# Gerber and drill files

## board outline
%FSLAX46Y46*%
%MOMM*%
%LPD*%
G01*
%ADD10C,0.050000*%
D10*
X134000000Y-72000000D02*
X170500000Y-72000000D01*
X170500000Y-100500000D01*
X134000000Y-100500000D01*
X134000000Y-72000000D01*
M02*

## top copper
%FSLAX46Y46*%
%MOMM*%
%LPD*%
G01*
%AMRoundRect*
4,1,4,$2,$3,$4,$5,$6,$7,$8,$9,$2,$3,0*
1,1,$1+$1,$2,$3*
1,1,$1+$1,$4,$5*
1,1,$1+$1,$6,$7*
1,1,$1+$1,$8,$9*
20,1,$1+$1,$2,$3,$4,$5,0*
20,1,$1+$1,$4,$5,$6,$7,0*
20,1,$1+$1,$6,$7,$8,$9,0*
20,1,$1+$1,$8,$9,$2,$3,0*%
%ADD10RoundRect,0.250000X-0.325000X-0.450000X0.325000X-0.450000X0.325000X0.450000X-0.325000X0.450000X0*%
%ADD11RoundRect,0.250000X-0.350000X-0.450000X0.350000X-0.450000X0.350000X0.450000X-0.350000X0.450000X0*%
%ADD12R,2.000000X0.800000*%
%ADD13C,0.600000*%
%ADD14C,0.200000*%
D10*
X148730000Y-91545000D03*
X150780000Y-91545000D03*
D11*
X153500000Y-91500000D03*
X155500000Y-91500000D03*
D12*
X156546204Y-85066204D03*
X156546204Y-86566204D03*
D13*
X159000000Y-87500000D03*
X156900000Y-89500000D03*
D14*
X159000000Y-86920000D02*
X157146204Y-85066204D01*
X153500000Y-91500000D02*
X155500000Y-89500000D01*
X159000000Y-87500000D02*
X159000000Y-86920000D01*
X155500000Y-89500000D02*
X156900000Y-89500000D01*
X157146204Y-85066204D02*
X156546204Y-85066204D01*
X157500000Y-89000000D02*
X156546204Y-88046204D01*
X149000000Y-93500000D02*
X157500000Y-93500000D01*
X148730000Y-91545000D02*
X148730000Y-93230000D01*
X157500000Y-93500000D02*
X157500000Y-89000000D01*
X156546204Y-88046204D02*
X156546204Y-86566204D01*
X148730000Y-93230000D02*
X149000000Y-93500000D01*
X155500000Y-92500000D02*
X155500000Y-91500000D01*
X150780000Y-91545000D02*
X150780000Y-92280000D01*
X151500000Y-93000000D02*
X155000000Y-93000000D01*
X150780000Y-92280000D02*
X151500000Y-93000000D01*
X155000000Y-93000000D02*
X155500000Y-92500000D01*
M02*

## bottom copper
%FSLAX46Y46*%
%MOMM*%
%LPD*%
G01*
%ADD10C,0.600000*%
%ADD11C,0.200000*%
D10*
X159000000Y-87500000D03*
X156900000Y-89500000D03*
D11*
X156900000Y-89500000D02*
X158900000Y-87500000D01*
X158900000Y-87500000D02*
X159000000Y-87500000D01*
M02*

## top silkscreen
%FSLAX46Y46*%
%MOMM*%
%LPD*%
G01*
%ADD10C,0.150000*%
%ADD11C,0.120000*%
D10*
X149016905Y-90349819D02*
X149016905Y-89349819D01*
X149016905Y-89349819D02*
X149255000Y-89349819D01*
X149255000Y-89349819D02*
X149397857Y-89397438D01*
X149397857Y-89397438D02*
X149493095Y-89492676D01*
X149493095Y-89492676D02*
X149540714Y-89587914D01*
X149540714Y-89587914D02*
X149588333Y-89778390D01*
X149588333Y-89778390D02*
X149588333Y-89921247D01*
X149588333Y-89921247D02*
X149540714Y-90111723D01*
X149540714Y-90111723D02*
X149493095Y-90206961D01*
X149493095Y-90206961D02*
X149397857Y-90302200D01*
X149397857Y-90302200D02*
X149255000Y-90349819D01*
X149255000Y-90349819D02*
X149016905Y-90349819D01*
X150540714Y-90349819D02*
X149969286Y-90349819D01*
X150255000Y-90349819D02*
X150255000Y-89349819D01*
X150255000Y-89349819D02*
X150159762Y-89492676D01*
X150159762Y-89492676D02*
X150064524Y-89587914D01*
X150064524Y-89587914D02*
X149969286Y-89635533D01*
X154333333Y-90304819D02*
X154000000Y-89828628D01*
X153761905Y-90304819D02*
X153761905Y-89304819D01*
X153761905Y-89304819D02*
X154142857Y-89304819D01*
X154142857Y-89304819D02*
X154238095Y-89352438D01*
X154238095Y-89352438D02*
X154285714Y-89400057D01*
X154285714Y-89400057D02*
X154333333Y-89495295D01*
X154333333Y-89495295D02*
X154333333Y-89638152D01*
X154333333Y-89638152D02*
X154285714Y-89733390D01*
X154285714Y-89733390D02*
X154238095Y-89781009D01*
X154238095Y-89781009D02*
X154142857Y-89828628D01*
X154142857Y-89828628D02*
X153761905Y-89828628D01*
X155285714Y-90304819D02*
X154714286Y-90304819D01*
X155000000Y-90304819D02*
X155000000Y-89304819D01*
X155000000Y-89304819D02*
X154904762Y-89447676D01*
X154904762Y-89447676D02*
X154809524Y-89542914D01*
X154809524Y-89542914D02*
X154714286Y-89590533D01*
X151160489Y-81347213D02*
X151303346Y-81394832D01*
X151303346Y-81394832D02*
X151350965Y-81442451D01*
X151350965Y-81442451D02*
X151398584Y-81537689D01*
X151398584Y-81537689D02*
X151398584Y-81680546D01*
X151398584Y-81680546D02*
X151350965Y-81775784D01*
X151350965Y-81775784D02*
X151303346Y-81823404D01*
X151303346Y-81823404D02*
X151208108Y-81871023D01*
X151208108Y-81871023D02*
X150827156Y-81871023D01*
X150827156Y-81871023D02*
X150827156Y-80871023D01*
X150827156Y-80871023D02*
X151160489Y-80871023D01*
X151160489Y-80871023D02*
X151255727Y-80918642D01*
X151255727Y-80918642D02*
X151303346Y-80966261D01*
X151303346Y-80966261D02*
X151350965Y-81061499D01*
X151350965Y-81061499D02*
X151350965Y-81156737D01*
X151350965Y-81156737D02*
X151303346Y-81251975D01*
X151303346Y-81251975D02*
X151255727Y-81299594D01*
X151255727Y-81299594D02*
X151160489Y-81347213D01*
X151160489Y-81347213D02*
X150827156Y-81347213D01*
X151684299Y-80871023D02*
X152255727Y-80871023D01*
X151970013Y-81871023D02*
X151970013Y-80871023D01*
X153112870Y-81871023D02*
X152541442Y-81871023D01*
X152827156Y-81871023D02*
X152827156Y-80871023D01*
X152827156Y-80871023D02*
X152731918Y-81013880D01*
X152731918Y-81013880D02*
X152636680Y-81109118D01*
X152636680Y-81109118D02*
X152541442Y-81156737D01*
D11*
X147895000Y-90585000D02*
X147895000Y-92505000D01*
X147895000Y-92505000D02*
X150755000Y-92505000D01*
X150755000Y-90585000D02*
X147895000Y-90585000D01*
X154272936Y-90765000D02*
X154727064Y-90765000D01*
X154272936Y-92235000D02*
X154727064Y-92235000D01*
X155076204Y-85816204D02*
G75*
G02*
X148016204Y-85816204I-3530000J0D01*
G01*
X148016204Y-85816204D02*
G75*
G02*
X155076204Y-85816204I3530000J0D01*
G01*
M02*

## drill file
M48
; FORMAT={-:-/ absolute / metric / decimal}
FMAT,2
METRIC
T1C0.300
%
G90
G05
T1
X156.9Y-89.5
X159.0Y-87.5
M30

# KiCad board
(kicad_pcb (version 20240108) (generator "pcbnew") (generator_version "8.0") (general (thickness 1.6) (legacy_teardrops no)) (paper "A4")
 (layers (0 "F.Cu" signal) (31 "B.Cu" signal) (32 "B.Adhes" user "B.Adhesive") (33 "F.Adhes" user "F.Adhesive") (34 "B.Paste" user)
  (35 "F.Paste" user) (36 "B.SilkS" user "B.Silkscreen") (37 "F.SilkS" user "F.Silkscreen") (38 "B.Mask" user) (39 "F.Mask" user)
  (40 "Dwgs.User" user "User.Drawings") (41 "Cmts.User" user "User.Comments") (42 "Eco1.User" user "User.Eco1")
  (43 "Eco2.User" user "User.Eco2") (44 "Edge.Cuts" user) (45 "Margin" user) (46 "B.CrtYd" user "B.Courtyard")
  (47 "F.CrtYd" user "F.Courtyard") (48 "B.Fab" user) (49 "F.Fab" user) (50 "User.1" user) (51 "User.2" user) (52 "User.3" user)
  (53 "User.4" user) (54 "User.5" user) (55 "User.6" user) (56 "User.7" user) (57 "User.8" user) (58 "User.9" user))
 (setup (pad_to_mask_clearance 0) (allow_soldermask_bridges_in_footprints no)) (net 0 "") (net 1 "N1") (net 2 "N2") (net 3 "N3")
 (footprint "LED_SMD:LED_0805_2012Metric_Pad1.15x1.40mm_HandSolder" (layer "F.Cu") (at 149.755 91.545)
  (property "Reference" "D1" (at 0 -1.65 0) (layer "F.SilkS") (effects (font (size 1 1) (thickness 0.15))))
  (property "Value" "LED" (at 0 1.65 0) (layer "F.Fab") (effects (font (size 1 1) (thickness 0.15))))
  (fp_line (start -1.86 -0.96) (end -1.86 0.96) (stroke (width 0.12) (type solid)) (layer "F.SilkS"))
  (fp_line (start -1.86 0.96) (end 1 0.96) (stroke (width 0.12) (type solid)) (layer "F.SilkS"))
  (fp_line (start 1 -0.96) (end -1.86 -0.96) (stroke (width 0.12) (type solid)) (layer "F.SilkS"))
  (pad "1" smd roundrect (at -1.025 0) (size 1.15 1.4) (layers "F.Cu" "F.Paste" "F.Mask") (roundrect_rratio 0.217391) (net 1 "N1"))
  (pad "2" smd roundrect (at 1.025 0) (size 1.15 1.4) (layers "F.Cu" "F.Paste" "F.Mask") (roundrect_rratio 0.217391) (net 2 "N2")))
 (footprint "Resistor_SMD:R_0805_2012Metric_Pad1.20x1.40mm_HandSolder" (layer "F.Cu") (at 154.5 91.5)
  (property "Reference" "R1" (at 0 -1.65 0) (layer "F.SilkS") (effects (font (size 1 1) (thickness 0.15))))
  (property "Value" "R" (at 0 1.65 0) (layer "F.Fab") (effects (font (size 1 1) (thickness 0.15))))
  (fp_line (start -0.227064 -0.735) (end 0.227064 -0.735) (stroke (width 0.12) (type solid)) (layer "F.SilkS"))
  (fp_line (start -0.227064 0.735) (end 0.227064 0.735) (stroke (width 0.12) (type solid)) (layer "F.SilkS"))
  (pad "1" smd roundrect (at -1 0) (size 1.2 1.4) (layers "F.Cu" "F.Paste" "F.Mask") (roundrect_rratio 0.208333) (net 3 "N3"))
  (pad "2" smd roundrect (at 1 0) (size 1.2 1.4) (layers "F.Cu" "F.Paste" "F.Mask") (roundrect_rratio 0.208333) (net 2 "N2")))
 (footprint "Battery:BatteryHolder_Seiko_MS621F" (layer "F.Cu") (at 156.546204 85.816204)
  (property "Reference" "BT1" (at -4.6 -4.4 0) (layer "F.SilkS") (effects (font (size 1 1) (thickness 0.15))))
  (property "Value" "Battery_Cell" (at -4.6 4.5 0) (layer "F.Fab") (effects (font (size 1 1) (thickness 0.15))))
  (fp_circle (center -5 0) (end -1.47 0) (stroke (width 0.12) (type solid)) (fill none) (layer "F.SilkS"))
  (pad "1" smd rect (at 0 -0.75) (size 2 0.8) (layers "F.Cu" "F.Paste" "F.Mask") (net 3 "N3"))
  (pad "2" smd rect (at 0 0.75) (size 2 0.8) (layers "F.Cu" "F.Paste" "F.Mask") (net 1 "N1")))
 (gr_rect (start 134 72) (end 170.5 100.5) (stroke (width 0.05) (type default)) (fill none) (layer "Edge.Cuts"))
 (segment (start 159 86.92) (end 157.146204 85.066204) (width 0.2) (layer "F.Cu") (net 3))
 (segment (start 153.5 91.5) (end 155.5 89.5) (width 0.2) (layer "F.Cu") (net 3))
 (segment (start 159 87.5) (end 159 86.92) (width 0.2) (layer "F.Cu") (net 3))
 (segment (start 155.5 89.5) (end 156.9 89.5) (width 0.2) (layer "F.Cu") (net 3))
 (segment (start 157.146204 85.066204) (end 156.546204 85.066204) (width 0.2) (layer "F.Cu") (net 3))
 (via (at 159 87.5) (size 0.6) (drill 0.3) (layers "F.Cu" "B.Cu") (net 3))
 (via (at 156.9 89.5) (size 0.6) (drill 0.3) (layers "F.Cu" "B.Cu") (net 3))
 (segment (start 156.9 89.5) (end 158.9 87.5) (width 0.2) (layer "B.Cu") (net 3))
 (segment (start 158.9 87.5) (end 159 87.5) (width 0.2) (layer "B.Cu") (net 3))
 (segment (start 157.5 89) (end 156.546204 88.046204) (width 0.2) (layer "F.Cu") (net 1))
 (segment (start 149 93.5) (end 157.5 93.5) (width 0.2) (layer "F.Cu") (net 1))
 (segment (start 148.73 91.545) (end 148.73 93.23) (width 0.2) (layer "F.Cu") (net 1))
 (segment (start 157.5 93.5) (end 157.5 89) (width 0.2) (layer "F.Cu") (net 1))
 (segment (start 156.546204 88.046204) (end 156.546204 86.566204) (width 0.2) (layer "F.Cu") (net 1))
 (segment (start 148.73 93.23) (end 149 93.5) (width 0.2) (layer "F.Cu") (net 1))
 (segment (start 155.5 92.5) (end 155.5 91.5) (width 0.2) (layer "F.Cu") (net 2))
 (segment (start 150.78 91.545) (end 150.78 92.28) (width 0.2) (layer "F.Cu") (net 2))
 (segment (start 151.5 93) (end 155 93) (width 0.2) (layer "F.Cu") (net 2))
 (segment (start 150.78 92.28) (end 151.5 93) (width 0.2) (layer "F.Cu") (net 2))
 (segment (start 155 93) (end 155.5 92.5) (width 0.2) (layer "F.Cu") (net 2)))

